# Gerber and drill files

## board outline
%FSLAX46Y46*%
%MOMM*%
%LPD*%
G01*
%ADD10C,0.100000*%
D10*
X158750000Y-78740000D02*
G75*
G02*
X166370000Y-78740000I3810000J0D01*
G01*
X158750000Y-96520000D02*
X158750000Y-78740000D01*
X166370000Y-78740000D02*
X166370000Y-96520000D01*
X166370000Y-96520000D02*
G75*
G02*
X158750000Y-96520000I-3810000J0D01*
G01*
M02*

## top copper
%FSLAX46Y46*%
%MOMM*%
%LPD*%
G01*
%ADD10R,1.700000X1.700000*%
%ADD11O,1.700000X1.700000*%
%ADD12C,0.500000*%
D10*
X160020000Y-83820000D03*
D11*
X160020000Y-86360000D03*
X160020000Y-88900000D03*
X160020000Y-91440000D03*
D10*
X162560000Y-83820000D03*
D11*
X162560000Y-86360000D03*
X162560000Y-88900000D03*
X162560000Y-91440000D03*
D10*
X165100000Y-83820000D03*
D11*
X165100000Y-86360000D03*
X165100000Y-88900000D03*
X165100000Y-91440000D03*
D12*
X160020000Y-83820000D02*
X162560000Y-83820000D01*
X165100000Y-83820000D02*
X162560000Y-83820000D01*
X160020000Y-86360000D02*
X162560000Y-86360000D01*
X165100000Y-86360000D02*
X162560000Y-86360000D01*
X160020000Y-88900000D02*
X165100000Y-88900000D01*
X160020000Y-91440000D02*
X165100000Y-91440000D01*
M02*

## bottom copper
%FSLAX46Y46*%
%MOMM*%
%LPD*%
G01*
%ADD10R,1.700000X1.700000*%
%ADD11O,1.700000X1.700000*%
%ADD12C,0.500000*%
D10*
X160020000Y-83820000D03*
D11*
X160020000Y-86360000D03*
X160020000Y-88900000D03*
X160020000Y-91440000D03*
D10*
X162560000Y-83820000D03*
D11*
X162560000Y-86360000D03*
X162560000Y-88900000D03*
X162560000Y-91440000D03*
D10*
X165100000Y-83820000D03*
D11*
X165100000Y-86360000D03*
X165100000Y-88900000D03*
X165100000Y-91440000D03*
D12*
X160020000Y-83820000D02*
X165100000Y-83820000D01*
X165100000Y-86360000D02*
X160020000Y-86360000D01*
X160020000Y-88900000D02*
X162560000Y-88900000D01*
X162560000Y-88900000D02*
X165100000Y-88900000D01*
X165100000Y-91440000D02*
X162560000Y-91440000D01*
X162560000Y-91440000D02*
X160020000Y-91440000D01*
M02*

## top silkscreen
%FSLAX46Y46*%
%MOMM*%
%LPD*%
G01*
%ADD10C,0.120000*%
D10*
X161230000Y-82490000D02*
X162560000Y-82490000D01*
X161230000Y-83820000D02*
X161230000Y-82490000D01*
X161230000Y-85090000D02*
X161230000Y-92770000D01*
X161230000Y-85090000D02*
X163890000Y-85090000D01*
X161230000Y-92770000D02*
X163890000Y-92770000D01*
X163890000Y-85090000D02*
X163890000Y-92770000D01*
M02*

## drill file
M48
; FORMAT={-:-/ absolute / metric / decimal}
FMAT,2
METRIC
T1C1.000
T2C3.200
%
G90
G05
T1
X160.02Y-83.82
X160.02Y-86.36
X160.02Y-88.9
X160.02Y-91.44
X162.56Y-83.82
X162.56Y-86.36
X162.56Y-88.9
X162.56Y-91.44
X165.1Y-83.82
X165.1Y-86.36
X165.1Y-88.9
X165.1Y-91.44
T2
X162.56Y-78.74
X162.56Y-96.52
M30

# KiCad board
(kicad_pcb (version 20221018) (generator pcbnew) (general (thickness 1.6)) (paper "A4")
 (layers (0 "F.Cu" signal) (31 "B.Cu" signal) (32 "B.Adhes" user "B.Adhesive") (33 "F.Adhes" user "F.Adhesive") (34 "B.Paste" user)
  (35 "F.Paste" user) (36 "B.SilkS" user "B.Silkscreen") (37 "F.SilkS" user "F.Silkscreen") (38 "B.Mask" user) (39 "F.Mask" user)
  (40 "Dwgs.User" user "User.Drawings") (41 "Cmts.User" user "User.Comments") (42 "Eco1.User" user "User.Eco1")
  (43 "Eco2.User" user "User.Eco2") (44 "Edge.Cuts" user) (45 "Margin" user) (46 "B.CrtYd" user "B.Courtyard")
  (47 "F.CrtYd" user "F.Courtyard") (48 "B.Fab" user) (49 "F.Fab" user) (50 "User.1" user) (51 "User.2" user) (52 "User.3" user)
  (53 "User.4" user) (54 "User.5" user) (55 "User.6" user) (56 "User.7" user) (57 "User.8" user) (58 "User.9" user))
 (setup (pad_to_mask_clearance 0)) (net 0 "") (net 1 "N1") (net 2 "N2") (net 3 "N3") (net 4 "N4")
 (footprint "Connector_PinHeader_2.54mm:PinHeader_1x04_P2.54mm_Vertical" (layer "F.Cu") (at 160.02 83.82)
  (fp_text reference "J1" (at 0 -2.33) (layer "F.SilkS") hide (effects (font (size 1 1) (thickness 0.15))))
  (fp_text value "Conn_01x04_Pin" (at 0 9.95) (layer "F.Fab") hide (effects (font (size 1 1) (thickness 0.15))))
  (pad "1" thru_hole rect (at 0 0) (size 1.7 1.7) (drill 1) (layers "*.Cu" "*.Mask") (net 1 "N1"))
  (pad "2" thru_hole oval (at 0 2.54) (size 1.7 1.7) (drill 1) (layers "*.Cu" "*.Mask") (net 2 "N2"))
  (pad "3" thru_hole oval (at 0 5.08) (size 1.7 1.7) (drill 1) (layers "*.Cu" "*.Mask") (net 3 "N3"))
  (pad "4" thru_hole oval (at 0 7.62) (size 1.7 1.7) (drill 1) (layers "*.Cu" "*.Mask") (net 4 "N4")))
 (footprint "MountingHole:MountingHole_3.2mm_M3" (layer "F.Cu") (at 162.56 78.74)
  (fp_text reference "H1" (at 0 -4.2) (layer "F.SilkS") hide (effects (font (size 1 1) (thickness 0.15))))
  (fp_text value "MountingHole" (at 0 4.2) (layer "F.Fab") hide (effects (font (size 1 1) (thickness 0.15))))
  (pad "" np_thru_hole circle (at 0 0) (size 3.2 3.2) (drill 3.2) (layers "*.Cu" "*.Mask")))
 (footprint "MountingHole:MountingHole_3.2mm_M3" (layer "F.Cu") (at 162.56 96.52)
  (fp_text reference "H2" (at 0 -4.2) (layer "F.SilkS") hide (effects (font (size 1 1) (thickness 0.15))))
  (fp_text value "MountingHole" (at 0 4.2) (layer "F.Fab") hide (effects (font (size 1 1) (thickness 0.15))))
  (pad "" np_thru_hole circle (at 0 0) (size 3.2 3.2) (drill 3.2) (layers "*.Cu" "*.Mask")))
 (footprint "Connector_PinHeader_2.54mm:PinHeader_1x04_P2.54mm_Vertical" (layer "F.Cu") (at 162.56 83.82)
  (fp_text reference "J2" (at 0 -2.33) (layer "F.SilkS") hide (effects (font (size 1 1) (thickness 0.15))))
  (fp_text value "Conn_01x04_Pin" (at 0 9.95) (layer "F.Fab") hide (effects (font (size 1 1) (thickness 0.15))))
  (fp_line (start -1.33 -1.33) (end 0 -1.33) (stroke (width 0.12) (type solid)) (layer "F.SilkS"))
  (fp_line (start -1.33 0) (end -1.33 -1.33) (stroke (width 0.12) (type solid)) (layer "F.SilkS"))
  (fp_line (start -1.33 1.27) (end -1.33 8.95) (stroke (width 0.12) (type solid)) (layer "F.SilkS"))
  (fp_line (start -1.33 1.27) (end 1.33 1.27) (stroke (width 0.12) (type solid)) (layer "F.SilkS"))
  (fp_line (start -1.33 8.95) (end 1.33 8.95) (stroke (width 0.12) (type solid)) (layer "F.SilkS"))
  (fp_line (start 1.33 1.27) (end 1.33 8.95) (stroke (width 0.12) (type solid)) (layer "F.SilkS"))
  (pad "1" thru_hole rect (at 0 0) (size 1.7 1.7) (drill 1) (layers "*.Cu" "*.Mask") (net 1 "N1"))
  (pad "2" thru_hole oval (at 0 2.54) (size 1.7 1.7) (drill 1) (layers "*.Cu" "*.Mask") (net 2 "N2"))
  (pad "3" thru_hole oval (at 0 5.08) (size 1.7 1.7) (drill 1) (layers "*.Cu" "*.Mask") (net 3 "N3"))
  (pad "4" thru_hole oval (at 0 7.62) (size 1.7 1.7) (drill 1) (layers "*.Cu" "*.Mask") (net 4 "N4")))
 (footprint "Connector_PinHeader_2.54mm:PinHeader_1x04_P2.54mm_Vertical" (layer "F.Cu") (at 165.1 83.82)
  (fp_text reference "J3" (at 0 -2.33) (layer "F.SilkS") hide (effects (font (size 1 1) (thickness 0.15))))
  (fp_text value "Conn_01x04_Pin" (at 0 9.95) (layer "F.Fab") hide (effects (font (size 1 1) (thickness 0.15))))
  (pad "1" thru_hole rect (at 0 0) (size 1.7 1.7) (drill 1) (layers "*.Cu" "*.Mask") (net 1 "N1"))
  (pad "2" thru_hole oval (at 0 2.54) (size 1.7 1.7) (drill 1) (layers "*.Cu" "*.Mask") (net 2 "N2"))
  (pad "3" thru_hole oval (at 0 5.08) (size 1.7 1.7) (drill 1) (layers "*.Cu" "*.Mask") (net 3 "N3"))
  (pad "4" thru_hole oval (at 0 7.62) (size 1.7 1.7) (drill 1) (layers "*.Cu" "*.Mask") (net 4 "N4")))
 (gr_arc (start 158.75 78.74) (mid 162.56 74.93) (end 166.37 78.74) (stroke (width 0.1) (type default)) (layer "Edge.Cuts"))
 (gr_line (start 158.75 96.52) (end 158.75 78.74) (stroke (width 0.1) (type default)) (layer "Edge.Cuts"))
 (gr_line (start 166.37 78.74) (end 166.37 96.52) (stroke (width 0.1) (type default)) (layer "Edge.Cuts"))
 (gr_arc (start 166.37 96.52) (mid 162.56 100.33) (end 158.75 96.52) (stroke (width 0.1) (type default)) (layer "Edge.Cuts"))
 (segment (start 160.02 83.82) (end 162.56 83.82) (width 0.5) (layer "F.Cu") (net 1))
 (segment (start 165.1 83.82) (end 162.56 83.82) (width 0.5) (layer "F.Cu") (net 1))
 (segment (start 160.02 83.82) (end 165.1 83.82) (width 0.5) (layer "B.Cu") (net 1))
 (segment (start 160.02 86.36) (end 162.56 86.36) (width 0.5) (layer "F.Cu") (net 2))
 (segment (start 165.1 86.36) (end 162.56 86.36) (width 0.5) (layer "F.Cu") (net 2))
 (segment (start 165.1 86.36) (end 160.02 86.36) (width 0.5) (layer "B.Cu") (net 2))
 (segment (start 160.02 88.9) (end 165.1 88.9) (width 0.5) (layer "F.Cu") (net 3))
 (segment (start 160.02 88.9) (end 162.56 88.9) (width 0.5) (layer "B.Cu") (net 3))
 (segment (start 162.56 88.9) (end 165.1 88.9) (width 0.5) (layer "B.Cu") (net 3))
 (segment (start 160.02 91.44) (end 165.1 91.44) (width 0.5) (layer "F.Cu") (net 4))
 (segment (start 165.1 91.44) (end 162.56 91.44) (width 0.5) (layer "B.Cu") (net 4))
 (segment (start 162.56 91.44) (end 160.02 91.44) (width 0.5) (layer "B.Cu") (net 4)))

